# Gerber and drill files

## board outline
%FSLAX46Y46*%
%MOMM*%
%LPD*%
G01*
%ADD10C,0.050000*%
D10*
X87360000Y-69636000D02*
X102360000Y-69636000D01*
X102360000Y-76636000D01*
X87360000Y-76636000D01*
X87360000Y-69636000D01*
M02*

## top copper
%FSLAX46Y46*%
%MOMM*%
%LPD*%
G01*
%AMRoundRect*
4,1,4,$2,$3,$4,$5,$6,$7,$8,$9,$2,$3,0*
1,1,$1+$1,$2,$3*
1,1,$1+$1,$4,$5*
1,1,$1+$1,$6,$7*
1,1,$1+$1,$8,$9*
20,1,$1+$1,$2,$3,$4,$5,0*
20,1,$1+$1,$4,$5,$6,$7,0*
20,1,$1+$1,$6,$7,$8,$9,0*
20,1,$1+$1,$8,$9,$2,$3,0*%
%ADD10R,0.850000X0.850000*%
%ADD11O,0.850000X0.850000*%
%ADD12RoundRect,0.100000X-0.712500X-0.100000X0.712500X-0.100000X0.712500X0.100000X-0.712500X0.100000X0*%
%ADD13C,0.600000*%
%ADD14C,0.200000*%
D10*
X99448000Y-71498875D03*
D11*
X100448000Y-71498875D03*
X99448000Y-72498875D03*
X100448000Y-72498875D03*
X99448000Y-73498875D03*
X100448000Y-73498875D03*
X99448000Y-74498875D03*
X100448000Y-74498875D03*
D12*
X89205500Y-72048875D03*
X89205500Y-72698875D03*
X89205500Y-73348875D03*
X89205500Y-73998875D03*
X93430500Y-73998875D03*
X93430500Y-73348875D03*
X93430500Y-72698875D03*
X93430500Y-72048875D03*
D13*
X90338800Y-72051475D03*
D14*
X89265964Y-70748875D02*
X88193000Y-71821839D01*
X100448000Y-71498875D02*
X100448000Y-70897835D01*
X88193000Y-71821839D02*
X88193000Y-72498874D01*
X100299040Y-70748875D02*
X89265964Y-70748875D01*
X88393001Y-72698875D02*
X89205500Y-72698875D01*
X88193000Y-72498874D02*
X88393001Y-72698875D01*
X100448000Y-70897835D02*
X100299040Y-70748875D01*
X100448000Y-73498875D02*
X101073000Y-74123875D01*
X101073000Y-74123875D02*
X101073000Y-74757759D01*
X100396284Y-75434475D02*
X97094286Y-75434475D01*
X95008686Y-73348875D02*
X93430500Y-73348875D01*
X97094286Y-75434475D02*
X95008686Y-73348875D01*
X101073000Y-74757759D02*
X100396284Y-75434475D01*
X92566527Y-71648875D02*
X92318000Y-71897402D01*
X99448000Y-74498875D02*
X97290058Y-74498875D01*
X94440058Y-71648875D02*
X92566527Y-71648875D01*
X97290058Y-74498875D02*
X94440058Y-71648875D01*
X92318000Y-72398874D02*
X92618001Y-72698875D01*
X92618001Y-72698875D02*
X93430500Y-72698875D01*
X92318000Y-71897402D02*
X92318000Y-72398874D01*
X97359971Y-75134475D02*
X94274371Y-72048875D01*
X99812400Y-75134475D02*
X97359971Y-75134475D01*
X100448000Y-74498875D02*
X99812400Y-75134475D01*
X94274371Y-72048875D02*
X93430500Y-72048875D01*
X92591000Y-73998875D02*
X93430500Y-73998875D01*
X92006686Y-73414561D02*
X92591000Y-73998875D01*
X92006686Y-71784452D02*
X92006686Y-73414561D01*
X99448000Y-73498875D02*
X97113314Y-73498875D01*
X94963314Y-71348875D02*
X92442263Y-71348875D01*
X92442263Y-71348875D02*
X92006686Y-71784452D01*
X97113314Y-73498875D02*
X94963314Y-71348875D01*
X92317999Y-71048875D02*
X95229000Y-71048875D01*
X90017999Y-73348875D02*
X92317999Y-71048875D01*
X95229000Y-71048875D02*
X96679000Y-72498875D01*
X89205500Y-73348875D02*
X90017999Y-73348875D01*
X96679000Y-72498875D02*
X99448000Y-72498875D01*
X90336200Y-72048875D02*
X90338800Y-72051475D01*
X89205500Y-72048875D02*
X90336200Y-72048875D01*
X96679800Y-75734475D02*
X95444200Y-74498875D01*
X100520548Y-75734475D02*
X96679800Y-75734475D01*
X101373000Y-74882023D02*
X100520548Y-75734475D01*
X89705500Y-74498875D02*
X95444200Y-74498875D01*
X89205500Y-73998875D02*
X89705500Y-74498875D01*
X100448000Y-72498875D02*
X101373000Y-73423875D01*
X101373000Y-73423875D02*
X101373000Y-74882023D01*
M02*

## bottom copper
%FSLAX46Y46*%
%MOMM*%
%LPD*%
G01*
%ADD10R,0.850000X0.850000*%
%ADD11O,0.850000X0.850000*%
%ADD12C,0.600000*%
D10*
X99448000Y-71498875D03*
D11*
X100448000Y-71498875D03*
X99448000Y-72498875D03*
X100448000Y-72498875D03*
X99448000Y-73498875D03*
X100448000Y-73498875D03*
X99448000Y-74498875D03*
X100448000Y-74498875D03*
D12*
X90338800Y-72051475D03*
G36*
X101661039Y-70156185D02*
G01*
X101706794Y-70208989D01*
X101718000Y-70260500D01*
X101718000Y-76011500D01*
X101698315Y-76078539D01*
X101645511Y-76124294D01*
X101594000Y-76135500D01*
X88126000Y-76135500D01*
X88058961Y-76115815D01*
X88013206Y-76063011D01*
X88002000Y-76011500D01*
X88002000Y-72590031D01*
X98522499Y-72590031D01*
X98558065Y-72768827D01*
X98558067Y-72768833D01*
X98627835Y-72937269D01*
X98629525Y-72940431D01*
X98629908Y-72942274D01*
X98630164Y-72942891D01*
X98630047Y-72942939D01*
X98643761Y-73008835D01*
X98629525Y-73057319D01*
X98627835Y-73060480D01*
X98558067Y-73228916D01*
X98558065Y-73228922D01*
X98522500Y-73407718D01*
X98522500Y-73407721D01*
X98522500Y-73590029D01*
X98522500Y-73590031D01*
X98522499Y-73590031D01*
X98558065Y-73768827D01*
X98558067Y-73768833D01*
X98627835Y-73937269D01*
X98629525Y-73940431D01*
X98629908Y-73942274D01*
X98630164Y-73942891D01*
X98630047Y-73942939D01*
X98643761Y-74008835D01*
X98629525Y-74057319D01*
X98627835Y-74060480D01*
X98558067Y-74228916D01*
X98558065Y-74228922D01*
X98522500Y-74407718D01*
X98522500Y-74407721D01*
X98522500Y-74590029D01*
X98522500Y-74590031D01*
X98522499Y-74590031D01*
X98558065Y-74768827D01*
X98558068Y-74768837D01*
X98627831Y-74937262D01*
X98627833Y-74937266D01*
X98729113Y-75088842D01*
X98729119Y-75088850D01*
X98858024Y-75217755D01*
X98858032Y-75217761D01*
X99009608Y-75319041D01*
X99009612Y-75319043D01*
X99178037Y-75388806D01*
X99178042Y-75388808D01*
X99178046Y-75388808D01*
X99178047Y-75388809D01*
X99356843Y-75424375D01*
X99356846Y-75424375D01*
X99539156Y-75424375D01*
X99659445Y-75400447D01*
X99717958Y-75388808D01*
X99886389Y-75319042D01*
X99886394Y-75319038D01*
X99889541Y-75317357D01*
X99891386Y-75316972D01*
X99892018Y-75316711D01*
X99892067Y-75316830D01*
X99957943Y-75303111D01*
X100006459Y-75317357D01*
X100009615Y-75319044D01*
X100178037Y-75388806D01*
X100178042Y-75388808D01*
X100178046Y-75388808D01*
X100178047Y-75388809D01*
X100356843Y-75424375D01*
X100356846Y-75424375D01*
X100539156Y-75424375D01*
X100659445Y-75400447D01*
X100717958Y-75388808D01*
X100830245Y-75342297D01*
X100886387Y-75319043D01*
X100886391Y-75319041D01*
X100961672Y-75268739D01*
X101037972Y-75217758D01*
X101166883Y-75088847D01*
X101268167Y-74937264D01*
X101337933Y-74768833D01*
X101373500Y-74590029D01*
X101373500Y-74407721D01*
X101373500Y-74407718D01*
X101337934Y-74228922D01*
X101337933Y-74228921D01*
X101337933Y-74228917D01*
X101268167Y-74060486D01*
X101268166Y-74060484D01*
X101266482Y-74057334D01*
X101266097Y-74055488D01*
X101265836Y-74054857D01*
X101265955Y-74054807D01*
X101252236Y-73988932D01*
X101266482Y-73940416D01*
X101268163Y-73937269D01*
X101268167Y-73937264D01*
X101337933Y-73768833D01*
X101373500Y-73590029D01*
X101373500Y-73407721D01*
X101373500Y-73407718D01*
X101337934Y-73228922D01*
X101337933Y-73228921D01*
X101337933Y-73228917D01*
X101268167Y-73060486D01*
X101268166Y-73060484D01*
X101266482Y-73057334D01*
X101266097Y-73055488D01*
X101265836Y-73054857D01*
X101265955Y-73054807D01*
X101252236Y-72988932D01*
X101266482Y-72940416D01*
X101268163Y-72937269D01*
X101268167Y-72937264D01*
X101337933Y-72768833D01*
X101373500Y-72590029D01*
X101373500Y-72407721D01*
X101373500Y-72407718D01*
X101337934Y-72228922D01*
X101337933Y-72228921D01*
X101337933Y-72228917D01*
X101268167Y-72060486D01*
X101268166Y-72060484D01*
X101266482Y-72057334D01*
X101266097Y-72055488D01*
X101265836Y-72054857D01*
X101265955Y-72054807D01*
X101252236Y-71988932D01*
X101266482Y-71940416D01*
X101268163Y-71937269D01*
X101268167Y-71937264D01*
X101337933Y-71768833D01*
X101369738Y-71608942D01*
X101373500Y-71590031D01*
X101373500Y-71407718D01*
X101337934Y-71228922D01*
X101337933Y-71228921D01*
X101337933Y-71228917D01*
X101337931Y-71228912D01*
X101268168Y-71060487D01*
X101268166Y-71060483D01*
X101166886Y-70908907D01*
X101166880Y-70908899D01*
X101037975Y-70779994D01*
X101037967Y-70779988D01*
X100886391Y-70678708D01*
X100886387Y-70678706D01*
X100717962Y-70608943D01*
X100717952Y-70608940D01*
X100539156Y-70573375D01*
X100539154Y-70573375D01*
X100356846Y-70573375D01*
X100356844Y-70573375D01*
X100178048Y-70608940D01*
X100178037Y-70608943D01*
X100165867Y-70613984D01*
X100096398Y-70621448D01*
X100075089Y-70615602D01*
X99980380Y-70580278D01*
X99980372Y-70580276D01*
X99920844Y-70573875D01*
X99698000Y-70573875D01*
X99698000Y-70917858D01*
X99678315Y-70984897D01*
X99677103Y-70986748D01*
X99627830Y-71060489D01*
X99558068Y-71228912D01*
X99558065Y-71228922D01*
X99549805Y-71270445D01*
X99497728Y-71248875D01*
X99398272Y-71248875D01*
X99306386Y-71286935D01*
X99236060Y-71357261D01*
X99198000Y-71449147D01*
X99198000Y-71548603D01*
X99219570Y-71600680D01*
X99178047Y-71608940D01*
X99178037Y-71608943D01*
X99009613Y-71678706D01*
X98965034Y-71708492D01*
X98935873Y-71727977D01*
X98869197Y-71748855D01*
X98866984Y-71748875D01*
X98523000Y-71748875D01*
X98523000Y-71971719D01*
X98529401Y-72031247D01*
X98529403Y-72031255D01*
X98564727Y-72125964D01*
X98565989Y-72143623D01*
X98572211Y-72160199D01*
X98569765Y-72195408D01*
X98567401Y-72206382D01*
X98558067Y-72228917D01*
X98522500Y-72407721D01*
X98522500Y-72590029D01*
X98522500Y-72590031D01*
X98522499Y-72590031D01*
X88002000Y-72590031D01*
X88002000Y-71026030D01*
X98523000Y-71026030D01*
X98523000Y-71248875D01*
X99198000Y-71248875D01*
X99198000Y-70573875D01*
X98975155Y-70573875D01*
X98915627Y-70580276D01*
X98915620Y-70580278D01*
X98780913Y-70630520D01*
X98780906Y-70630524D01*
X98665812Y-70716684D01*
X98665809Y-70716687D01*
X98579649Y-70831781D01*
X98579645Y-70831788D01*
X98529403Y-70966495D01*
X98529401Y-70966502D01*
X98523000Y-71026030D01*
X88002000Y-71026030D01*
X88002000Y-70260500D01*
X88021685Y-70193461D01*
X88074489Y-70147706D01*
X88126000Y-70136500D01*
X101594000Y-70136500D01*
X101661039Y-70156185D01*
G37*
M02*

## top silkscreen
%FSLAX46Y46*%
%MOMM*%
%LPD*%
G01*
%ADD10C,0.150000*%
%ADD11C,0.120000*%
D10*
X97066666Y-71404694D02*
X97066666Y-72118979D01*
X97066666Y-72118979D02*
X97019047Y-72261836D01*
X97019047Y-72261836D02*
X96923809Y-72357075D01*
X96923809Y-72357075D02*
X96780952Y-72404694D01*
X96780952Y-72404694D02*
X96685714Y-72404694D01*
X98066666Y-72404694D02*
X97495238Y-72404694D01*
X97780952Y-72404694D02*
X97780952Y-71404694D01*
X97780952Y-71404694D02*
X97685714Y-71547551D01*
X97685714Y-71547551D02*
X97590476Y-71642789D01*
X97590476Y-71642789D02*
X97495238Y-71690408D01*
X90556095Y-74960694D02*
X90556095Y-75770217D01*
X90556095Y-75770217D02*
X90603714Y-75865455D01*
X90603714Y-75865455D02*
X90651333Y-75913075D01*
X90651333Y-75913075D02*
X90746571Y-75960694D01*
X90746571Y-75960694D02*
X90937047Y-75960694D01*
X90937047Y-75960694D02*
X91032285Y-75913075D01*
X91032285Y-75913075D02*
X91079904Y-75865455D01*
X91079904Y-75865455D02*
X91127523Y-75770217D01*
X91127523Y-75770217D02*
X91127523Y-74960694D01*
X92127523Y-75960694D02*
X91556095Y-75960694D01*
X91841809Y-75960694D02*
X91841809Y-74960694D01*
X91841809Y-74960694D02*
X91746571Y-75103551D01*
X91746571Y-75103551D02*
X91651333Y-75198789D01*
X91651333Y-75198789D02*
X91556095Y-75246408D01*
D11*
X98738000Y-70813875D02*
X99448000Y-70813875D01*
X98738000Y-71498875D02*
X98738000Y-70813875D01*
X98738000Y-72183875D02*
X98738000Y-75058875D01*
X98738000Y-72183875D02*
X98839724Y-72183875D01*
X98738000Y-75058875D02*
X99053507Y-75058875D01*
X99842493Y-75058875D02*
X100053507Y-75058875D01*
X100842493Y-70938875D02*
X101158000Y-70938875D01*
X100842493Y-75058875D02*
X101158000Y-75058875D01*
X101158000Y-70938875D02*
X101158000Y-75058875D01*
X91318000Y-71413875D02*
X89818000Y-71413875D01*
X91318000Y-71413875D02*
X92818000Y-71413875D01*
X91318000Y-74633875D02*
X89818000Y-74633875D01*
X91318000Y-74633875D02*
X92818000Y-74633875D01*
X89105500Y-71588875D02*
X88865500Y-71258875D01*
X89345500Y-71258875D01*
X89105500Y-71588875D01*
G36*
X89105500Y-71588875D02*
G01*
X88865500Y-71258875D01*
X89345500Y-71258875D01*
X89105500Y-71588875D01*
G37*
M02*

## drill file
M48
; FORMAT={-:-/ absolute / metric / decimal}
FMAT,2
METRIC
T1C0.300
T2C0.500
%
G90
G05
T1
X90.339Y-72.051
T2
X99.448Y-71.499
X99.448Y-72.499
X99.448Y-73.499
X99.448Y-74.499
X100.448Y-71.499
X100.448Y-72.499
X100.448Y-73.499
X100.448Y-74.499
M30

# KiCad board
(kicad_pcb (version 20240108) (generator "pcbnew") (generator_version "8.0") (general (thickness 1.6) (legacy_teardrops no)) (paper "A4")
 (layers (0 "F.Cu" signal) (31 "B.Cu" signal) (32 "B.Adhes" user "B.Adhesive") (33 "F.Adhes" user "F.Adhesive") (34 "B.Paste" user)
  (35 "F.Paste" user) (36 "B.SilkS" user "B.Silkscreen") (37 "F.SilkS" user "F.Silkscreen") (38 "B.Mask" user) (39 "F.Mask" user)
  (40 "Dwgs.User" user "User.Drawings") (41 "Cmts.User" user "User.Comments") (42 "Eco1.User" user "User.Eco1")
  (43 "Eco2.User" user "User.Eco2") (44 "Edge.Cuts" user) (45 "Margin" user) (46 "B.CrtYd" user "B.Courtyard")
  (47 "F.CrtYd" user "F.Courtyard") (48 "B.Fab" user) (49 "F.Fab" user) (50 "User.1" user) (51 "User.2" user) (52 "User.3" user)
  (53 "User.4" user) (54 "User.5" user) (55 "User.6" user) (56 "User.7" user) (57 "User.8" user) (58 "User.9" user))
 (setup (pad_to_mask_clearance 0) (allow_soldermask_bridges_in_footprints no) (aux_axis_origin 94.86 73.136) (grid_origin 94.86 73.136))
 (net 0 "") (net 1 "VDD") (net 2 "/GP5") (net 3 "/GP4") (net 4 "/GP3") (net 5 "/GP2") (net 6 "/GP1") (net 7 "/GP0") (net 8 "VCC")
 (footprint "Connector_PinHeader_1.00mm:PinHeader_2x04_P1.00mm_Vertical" (layer "F.Cu") (at 99.448 71.498875)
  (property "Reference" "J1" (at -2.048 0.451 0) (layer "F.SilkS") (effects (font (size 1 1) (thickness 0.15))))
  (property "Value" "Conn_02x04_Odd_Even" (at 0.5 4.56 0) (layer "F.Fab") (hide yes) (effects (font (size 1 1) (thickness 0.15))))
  (fp_line (start -0.71 -0.685) (end 0 -0.685) (stroke (width 0.12) (type solid)) (layer "F.SilkS"))
  (fp_line (start -0.71 0) (end -0.71 -0.685) (stroke (width 0.12) (type solid)) (layer "F.SilkS"))
  (fp_line (start -0.71 0.685) (end -0.71 3.56) (stroke (width 0.12) (type solid)) (layer "F.SilkS"))
  (fp_line (start -0.71 0.685) (end -0.608276 0.685) (stroke (width 0.12) (type solid)) (layer "F.SilkS"))
  (fp_line (start -0.71 3.56) (end -0.394493 3.56) (stroke (width 0.12) (type solid)) (layer "F.SilkS"))
  (fp_line (start 0.394493 3.56) (end 0.605507 3.56) (stroke (width 0.12) (type solid)) (layer "F.SilkS"))
  (fp_line (start 1.394493 -0.56) (end 1.71 -0.56) (stroke (width 0.12) (type solid)) (layer "F.SilkS"))
  (fp_line (start 1.394493 3.56) (end 1.71 3.56) (stroke (width 0.12) (type solid)) (layer "F.SilkS"))
  (fp_line (start 1.71 -0.56) (end 1.71 3.56) (stroke (width 0.12) (type solid)) (layer "F.SilkS"))
  (pad "1" thru_hole rect (at 0 0) (size 0.85 0.85) (drill 0.5) (layers "*.Cu" "*.Mask") (remove_unused_layers no) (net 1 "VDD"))
  (pad "2" thru_hole oval (at 1 0) (size 0.85 0.85) (drill 0.5) (layers "*.Cu" "*.Mask") (remove_unused_layers no) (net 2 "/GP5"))
  (pad "3" thru_hole oval (at 0 1) (size 0.85 0.85) (drill 0.5) (layers "*.Cu" "*.Mask") (remove_unused_layers no) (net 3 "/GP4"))
  (pad "4" thru_hole oval (at 1 1) (size 0.85 0.85) (drill 0.5) (layers "*.Cu" "*.Mask") (remove_unused_layers no) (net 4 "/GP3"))
  (pad "5" thru_hole oval (at 0 2) (size 0.85 0.85) (drill 0.5) (layers "*.Cu" "*.Mask") (remove_unused_layers no) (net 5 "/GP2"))
  (pad "6" thru_hole oval (at 1 2) (size 0.85 0.85) (drill 0.5) (layers "*.Cu" "*.Mask") (remove_unused_layers no) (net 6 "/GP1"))
  (pad "7" thru_hole oval (at 0 3) (size 0.85 0.85) (drill 0.5) (layers "*.Cu" "*.Mask") (remove_unused_layers no) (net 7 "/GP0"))
  (pad "8" thru_hole oval (at 1 3) (size 0.85 0.85) (drill 0.5) (layers "*.Cu" "*.Mask") (remove_unused_layers no) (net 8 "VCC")))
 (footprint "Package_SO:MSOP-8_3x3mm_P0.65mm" (layer "F.Cu") (at 91.318 73.023875)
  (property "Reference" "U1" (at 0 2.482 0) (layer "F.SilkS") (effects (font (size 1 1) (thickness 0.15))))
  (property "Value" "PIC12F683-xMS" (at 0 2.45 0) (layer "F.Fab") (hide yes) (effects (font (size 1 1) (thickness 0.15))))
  (fp_line (start 0 -1.61) (end -1.5 -1.61) (stroke (width 0.12) (type solid)) (layer "F.SilkS"))
  (fp_line (start 0 -1.61) (end 1.5 -1.61) (stroke (width 0.12) (type solid)) (layer "F.SilkS"))
  (fp_line (start 0 1.61) (end -1.5 1.61) (stroke (width 0.12) (type solid)) (layer "F.SilkS"))
  (fp_line (start 0 1.61) (end 1.5 1.61) (stroke (width 0.12) (type solid)) (layer "F.SilkS"))
  (fp_poly
   (pts (xy -2.2125 -1.435) (xy -2.4525 -1.765) (xy -1.9725 -1.765) (xy -2.2125 -1.435)) (stroke (width 0.12) (type solid)) (fill solid)
   (layer "F.SilkS"))
  (pad "1" smd roundrect (at -2.1125 -0.975) (size 1.625 0.4) (layers "F.Cu" "F.Paste" "F.Mask") (roundrect_rratio 0.25) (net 1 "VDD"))
  (pad "2" smd roundrect (at -2.1125 -0.325) (size 1.625 0.4) (layers "F.Cu" "F.Paste" "F.Mask") (roundrect_rratio 0.25) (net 2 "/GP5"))
  (pad "3" smd roundrect (at -2.1125 0.325) (size 1.625 0.4) (layers "F.Cu" "F.Paste" "F.Mask") (roundrect_rratio 0.25) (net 3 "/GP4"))
  (pad "4" smd roundrect (at -2.1125 0.975) (size 1.625 0.4) (layers "F.Cu" "F.Paste" "F.Mask") (roundrect_rratio 0.25) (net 4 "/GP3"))
  (pad "5" smd roundrect (at 2.1125 0.975) (size 1.625 0.4) (layers "F.Cu" "F.Paste" "F.Mask") (roundrect_rratio 0.25) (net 5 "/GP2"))
  (pad "6" smd roundrect (at 2.1125 0.325) (size 1.625 0.4) (layers "F.Cu" "F.Paste" "F.Mask") (roundrect_rratio 0.25) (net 6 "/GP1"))
  (pad "7" smd roundrect (at 2.1125 -0.325) (size 1.625 0.4) (layers "F.Cu" "F.Paste" "F.Mask") (roundrect_rratio 0.25) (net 7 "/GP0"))
  (pad "8" smd roundrect (at 2.1125 -0.975) (size 1.625 0.4) (layers "F.Cu" "F.Paste" "F.Mask") (roundrect_rratio 0.25) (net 8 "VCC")))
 (gr_rect (start 87.36 69.636) (end 102.36 76.636) (stroke (width 0.05) (type default)) (fill none) (layer "Edge.Cuts"))
 (segment (start 89.265964 70.748875) (end 88.193 71.821839) (width 0.2) (layer "F.Cu") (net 2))
 (segment (start 100.448 71.498875) (end 100.448 70.897835) (width 0.2) (layer "F.Cu") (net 2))
 (segment (start 88.193 71.821839) (end 88.193 72.498874) (width 0.2) (layer "F.Cu") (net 2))
 (segment (start 100.29904 70.748875) (end 89.265964 70.748875) (width 0.2) (layer "F.Cu") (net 2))
 (segment (start 88.393001 72.698875) (end 89.2055 72.698875) (width 0.2) (layer "F.Cu") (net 2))
 (segment (start 88.193 72.498874) (end 88.393001 72.698875) (width 0.2) (layer "F.Cu") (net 2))
 (segment (start 100.448 70.897835) (end 100.29904 70.748875) (width 0.2) (layer "F.Cu") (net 2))
 (segment (start 100.448 73.498875) (end 101.073 74.123875) (width 0.2) (layer "F.Cu") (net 6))
 (segment (start 101.073 74.123875) (end 101.073 74.757759) (width 0.2) (layer "F.Cu") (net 6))
 (segment (start 100.396284 75.434475) (end 97.094286 75.434475) (width 0.2) (layer "F.Cu") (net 6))
 (segment (start 95.008686 73.348875) (end 93.4305 73.348875) (width 0.2) (layer "F.Cu") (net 6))
 (segment (start 97.094286 75.434475) (end 95.008686 73.348875) (width 0.2) (layer "F.Cu") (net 6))
 (segment (start 101.073 74.757759) (end 100.396284 75.434475) (width 0.2) (layer "F.Cu") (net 6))
 (segment (start 92.566527 71.648875) (end 92.318 71.897402) (width 0.2) (layer "F.Cu") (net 7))
 (segment (start 99.448 74.498875) (end 97.290058 74.498875) (width 0.2) (layer "F.Cu") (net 7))
 (segment (start 94.440058 71.648875) (end 92.566527 71.648875) (width 0.2) (layer "F.Cu") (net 7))
 (segment (start 97.290058 74.498875) (end 94.440058 71.648875) (width 0.2) (layer "F.Cu") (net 7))
 (segment (start 92.318 72.398874) (end 92.618001 72.698875) (width 0.2) (layer "F.Cu") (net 7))
 (segment (start 92.618001 72.698875) (end 93.4305 72.698875) (width 0.2) (layer "F.Cu") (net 7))
 (segment (start 92.318 71.897402) (end 92.318 72.398874) (width 0.2) (layer "F.Cu") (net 7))
 (segment (start 97.359971 75.134475) (end 94.274371 72.048875) (width 0.2) (layer "F.Cu") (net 8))
 (segment (start 99.8124 75.134475) (end 97.359971 75.134475) (width 0.2) (layer "F.Cu") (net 8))
 (segment (start 100.448 74.498875) (end 99.8124 75.134475) (width 0.2) (layer "F.Cu") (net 8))
 (segment (start 94.274371 72.048875) (end 93.4305 72.048875) (width 0.2) (layer "F.Cu") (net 8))
 (segment (start 92.591 73.998875) (end 93.4305 73.998875) (width 0.2) (layer "F.Cu") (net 5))
 (segment (start 92.006686 73.414561) (end 92.591 73.998875) (width 0.2) (layer "F.Cu") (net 5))
 (segment (start 92.006686 71.784452) (end 92.006686 73.414561) (width 0.2) (layer "F.Cu") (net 5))
 (segment (start 99.448 73.498875) (end 97.113314 73.498875) (width 0.2) (layer "F.Cu") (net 5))
 (segment (start 94.963314 71.348875) (end 92.442263 71.348875) (width 0.2) (layer "F.Cu") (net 5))
 (segment (start 92.442263 71.348875) (end 92.006686 71.784452) (width 0.2) (layer "F.Cu") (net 5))
 (segment (start 97.113314 73.498875) (end 94.963314 71.348875) (width 0.2) (layer "F.Cu") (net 5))
 (segment (start 92.317999 71.048875) (end 95.229 71.048875) (width 0.2) (layer "F.Cu") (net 3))
 (segment (start 90.017999 73.348875) (end 92.317999 71.048875) (width 0.2) (layer "F.Cu") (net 3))
 (segment (start 95.229 71.048875) (end 96.679 72.498875) (width 0.2) (layer "F.Cu") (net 3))
 (segment (start 89.2055 73.348875) (end 90.017999 73.348875) (width 0.2) (layer "F.Cu") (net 3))
 (segment (start 96.679 72.498875) (end 99.448 72.498875) (width 0.2) (layer "F.Cu") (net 3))
 (segment (start 90.3362 72.048875) (end 90.3388 72.051475) (width 0.2) (layer "F.Cu") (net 1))
 (segment (start 89.2055 72.048875) (end 90.3362 72.048875) (width 0.2) (layer "F.Cu") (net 1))
 (via (at 90.3388 72.051475) (size 0.6) (drill 0.3) (layers "F.Cu" "B.Cu") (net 1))
 (segment (start 96.6798 75.734475) (end 95.4442 74.498875) (width 0.2) (layer "F.Cu") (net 4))
 (segment (start 100.520548 75.734475) (end 96.6798 75.734475) (width 0.2) (layer "F.Cu") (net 4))
 (segment (start 101.373 74.882023) (end 100.520548 75.734475) (width 0.2) (layer "F.Cu") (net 4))
 (segment (start 89.7055 74.498875) (end 95.4442 74.498875) (width 0.2) (layer "F.Cu") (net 4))
 (segment (start 89.2055 73.998875) (end 89.7055 74.498875) (width 0.2) (layer "F.Cu") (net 4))
 (segment (start 100.448 72.498875) (end 101.373 73.423875) (width 0.2) (layer "F.Cu") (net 4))
 (segment (start 101.373 73.423875) (end 101.373 74.882023) (width 0.2) (layer "F.Cu") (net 4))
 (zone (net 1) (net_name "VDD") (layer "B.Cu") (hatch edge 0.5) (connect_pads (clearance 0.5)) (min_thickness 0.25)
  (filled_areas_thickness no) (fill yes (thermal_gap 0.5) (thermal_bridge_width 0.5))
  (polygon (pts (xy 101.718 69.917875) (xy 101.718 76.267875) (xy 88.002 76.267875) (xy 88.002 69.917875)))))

